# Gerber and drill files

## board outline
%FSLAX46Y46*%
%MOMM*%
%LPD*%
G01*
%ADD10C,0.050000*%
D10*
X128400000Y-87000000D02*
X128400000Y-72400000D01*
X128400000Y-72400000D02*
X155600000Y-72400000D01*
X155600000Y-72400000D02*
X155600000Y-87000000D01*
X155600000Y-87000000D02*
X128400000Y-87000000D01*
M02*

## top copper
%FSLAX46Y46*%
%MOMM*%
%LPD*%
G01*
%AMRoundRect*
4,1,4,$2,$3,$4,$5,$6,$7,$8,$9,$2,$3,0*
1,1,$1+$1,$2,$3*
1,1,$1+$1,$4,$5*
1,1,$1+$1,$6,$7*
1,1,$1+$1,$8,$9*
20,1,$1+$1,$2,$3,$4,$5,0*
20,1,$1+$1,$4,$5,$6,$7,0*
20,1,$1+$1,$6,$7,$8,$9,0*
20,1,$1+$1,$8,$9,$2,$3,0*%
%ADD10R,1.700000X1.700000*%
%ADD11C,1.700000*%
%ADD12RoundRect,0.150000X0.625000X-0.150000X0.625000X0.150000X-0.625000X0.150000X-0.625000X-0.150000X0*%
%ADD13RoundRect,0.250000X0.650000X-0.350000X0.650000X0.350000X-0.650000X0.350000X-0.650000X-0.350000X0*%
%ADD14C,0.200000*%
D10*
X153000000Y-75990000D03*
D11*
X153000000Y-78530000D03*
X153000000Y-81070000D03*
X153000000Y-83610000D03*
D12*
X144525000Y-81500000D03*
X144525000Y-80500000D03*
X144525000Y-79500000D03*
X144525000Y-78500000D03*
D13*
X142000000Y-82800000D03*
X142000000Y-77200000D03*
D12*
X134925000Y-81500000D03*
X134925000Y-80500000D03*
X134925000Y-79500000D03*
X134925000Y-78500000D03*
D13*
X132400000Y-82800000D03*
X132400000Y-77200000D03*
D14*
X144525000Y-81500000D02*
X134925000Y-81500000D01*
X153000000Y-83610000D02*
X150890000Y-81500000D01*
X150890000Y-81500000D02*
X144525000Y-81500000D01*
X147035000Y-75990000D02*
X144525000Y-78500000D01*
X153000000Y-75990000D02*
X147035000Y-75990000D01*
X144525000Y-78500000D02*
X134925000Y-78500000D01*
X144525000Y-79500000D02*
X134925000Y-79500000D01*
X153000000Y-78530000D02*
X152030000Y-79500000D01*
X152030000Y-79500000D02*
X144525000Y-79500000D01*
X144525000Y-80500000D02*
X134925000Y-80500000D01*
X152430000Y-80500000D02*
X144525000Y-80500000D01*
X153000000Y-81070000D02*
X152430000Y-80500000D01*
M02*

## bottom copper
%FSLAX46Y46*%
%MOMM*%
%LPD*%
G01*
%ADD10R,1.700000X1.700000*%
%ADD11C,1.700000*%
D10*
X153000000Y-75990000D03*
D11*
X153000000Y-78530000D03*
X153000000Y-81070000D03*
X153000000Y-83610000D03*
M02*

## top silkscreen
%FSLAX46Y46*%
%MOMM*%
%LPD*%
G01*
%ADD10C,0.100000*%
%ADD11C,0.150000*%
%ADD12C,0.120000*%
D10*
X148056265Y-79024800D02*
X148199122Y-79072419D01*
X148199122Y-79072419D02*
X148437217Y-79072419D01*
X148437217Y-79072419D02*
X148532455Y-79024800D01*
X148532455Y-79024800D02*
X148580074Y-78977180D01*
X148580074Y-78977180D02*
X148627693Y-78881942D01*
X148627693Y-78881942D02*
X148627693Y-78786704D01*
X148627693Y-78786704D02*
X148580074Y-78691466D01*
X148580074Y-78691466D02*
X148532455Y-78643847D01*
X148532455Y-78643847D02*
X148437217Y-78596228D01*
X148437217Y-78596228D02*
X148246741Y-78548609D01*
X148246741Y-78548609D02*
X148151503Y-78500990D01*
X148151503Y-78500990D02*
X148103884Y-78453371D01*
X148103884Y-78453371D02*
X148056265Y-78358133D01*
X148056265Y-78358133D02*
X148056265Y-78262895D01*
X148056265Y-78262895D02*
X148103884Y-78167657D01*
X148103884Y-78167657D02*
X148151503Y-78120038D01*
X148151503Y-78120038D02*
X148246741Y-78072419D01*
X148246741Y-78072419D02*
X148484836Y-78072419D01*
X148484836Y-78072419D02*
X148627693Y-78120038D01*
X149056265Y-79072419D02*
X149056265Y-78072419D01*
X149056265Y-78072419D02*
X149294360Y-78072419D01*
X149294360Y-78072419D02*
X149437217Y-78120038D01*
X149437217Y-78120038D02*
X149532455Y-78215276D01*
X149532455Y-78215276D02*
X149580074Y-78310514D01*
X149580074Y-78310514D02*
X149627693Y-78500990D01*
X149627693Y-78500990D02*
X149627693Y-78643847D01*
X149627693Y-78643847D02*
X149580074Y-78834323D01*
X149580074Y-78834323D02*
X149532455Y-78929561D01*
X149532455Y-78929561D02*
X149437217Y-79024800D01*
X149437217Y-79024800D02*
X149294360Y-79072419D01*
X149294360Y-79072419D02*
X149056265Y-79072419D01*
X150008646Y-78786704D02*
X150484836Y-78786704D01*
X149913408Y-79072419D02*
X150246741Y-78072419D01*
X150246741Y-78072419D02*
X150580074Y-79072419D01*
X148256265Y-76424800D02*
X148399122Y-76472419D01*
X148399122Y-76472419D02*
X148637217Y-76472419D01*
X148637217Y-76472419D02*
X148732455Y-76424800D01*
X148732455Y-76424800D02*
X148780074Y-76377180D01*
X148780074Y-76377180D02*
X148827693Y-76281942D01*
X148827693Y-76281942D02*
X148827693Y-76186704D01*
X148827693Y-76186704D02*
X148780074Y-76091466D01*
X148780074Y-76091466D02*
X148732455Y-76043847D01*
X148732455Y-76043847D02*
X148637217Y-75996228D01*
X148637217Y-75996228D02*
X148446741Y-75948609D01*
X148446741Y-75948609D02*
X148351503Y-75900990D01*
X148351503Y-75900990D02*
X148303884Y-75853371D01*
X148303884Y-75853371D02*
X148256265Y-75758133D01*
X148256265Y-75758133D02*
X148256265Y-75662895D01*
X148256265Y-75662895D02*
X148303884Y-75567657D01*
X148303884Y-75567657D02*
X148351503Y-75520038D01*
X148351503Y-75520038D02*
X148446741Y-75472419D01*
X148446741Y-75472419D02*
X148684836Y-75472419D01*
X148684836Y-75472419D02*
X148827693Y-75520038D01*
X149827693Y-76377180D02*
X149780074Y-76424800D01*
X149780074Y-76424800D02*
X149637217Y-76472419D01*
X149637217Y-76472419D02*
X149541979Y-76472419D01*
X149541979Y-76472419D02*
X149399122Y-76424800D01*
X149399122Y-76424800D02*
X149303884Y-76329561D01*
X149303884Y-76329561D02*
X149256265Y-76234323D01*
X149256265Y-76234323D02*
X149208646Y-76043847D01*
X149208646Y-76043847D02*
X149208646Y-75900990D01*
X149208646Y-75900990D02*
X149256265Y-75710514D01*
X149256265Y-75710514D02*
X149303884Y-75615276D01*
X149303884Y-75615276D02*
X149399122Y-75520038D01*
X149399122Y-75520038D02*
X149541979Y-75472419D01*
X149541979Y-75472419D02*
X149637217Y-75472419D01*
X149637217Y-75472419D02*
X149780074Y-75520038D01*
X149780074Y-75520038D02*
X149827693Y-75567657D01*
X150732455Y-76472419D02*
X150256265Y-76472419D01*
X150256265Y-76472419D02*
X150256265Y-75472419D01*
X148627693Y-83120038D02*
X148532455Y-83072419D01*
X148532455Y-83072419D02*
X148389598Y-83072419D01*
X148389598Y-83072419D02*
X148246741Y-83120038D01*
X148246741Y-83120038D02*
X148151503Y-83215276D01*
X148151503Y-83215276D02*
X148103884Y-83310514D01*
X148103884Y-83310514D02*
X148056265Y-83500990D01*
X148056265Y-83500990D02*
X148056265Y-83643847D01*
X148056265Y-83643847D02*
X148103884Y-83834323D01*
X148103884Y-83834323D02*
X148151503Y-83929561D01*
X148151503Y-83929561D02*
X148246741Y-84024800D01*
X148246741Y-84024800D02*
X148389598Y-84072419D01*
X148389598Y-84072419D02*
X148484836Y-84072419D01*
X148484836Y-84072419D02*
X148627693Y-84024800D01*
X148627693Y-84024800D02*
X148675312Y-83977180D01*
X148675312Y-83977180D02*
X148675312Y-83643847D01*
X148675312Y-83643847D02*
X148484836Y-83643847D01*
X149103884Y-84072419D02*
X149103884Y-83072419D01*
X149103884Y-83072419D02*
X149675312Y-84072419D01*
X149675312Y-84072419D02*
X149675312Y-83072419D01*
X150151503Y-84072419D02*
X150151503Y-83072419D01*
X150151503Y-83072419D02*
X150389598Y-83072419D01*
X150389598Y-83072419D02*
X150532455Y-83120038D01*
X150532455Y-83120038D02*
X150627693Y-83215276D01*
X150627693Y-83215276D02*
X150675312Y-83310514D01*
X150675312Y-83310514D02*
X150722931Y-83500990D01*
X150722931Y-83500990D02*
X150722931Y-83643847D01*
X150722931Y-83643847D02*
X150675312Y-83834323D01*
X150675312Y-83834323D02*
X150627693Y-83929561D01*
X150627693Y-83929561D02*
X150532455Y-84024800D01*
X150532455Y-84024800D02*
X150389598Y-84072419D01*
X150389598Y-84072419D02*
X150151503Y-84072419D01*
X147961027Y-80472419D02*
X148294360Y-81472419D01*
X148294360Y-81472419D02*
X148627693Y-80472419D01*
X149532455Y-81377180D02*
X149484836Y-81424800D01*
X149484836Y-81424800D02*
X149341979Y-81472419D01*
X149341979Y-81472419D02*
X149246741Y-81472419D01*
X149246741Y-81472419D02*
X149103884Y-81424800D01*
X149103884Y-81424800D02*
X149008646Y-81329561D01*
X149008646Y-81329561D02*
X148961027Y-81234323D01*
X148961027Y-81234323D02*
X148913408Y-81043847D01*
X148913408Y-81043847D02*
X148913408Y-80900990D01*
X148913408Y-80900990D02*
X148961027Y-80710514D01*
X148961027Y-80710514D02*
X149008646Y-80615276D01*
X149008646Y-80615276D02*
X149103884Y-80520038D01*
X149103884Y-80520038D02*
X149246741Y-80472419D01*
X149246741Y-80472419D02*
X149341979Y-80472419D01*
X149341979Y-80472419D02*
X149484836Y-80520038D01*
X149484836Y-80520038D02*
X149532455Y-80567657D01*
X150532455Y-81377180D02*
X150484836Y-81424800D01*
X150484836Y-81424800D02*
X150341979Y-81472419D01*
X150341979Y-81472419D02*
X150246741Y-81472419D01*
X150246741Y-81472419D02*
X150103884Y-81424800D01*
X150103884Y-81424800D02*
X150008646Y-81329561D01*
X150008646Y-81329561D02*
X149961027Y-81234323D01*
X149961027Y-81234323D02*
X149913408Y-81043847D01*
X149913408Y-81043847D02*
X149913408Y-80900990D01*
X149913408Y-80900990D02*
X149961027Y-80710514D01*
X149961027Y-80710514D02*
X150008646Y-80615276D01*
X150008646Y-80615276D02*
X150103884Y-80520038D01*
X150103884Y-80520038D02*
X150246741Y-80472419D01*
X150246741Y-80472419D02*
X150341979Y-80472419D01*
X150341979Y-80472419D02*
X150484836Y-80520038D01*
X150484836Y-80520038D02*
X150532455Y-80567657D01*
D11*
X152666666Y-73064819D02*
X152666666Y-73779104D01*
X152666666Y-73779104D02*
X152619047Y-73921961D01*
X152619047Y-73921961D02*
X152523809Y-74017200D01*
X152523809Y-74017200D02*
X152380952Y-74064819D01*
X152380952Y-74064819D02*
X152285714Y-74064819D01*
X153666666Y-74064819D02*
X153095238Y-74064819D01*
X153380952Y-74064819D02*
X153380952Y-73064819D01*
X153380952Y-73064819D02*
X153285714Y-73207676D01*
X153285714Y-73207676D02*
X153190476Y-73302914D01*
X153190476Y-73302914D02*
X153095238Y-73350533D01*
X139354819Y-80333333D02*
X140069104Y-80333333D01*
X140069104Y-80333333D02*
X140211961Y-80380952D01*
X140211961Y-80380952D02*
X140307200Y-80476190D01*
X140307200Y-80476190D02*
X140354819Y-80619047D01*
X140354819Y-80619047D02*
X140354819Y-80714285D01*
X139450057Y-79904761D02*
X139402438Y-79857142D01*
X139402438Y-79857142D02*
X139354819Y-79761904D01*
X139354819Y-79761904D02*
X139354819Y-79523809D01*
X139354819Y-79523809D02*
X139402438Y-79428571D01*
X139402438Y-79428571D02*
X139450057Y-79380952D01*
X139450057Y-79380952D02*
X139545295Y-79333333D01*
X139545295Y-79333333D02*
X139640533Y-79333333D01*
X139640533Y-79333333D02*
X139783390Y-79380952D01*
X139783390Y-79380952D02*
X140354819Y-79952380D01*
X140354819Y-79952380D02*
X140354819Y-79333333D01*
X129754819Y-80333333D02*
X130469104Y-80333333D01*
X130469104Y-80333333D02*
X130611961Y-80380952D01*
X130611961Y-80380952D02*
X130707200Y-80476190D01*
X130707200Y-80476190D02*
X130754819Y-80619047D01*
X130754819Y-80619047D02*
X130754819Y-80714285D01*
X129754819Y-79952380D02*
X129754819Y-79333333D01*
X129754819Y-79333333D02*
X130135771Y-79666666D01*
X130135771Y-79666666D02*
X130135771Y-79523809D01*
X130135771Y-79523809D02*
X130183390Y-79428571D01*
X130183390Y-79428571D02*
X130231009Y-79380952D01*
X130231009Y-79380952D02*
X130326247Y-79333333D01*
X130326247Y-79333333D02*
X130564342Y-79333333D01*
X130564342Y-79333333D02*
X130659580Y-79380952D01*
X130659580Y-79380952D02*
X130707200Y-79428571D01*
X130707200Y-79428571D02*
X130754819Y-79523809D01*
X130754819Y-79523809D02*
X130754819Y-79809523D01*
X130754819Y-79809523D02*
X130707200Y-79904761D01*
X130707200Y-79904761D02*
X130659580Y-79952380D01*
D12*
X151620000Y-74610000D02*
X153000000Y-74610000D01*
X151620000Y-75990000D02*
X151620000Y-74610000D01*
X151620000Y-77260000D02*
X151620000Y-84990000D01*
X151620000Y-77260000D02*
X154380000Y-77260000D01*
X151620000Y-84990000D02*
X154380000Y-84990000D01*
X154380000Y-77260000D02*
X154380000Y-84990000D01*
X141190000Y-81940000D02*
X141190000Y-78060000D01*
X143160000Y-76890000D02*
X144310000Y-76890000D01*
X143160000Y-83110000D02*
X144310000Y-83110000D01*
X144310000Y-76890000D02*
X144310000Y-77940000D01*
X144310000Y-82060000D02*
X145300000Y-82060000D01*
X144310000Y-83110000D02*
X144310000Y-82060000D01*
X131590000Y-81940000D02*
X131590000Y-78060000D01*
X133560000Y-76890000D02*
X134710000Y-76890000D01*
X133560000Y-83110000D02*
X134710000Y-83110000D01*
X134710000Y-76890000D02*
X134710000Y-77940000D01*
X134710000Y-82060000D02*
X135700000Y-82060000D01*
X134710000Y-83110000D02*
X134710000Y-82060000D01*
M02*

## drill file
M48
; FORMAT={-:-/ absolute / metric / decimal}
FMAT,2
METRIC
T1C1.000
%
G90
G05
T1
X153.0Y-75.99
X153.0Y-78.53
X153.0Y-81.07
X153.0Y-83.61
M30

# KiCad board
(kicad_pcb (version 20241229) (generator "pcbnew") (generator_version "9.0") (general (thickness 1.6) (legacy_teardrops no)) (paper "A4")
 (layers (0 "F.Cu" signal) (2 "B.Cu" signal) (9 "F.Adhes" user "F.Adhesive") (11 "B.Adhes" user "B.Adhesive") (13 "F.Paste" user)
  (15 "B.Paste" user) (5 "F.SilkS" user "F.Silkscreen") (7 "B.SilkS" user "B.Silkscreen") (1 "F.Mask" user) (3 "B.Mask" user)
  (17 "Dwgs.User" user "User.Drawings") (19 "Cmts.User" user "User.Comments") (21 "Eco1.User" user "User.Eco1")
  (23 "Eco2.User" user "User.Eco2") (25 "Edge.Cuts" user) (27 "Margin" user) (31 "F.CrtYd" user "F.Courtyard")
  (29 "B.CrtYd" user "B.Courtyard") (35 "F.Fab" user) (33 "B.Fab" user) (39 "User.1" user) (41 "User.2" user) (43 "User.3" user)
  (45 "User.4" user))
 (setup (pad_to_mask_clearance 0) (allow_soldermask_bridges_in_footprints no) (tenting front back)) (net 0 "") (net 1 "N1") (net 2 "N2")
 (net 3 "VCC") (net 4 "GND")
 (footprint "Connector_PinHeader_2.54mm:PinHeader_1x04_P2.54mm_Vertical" (layer "F.Cu") (at 153 75.99)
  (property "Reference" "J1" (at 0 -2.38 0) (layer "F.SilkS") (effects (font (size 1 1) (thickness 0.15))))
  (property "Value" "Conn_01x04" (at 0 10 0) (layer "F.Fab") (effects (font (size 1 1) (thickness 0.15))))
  (fp_line (start -1.38 -1.38) (end 0 -1.38) (stroke (width 0.12) (type solid)) (layer "F.SilkS"))
  (fp_line (start -1.38 0) (end -1.38 -1.38) (stroke (width 0.12) (type solid)) (layer "F.SilkS"))
  (fp_line (start -1.38 1.27) (end -1.38 9) (stroke (width 0.12) (type solid)) (layer "F.SilkS"))
  (fp_line (start -1.38 1.27) (end 1.38 1.27) (stroke (width 0.12) (type solid)) (layer "F.SilkS"))
  (fp_line (start -1.38 9) (end 1.38 9) (stroke (width 0.12) (type solid)) (layer "F.SilkS"))
  (fp_line (start 1.38 1.27) (end 1.38 9) (stroke (width 0.12) (type solid)) (layer "F.SilkS"))
  (pad "1" thru_hole rect (at 0 0) (size 1.7 1.7) (drill 1) (layers "*.Cu" "*.Mask") (remove_unused_layers no) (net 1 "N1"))
  (pad "2" thru_hole circle (at 0 2.54) (size 1.7 1.7) (drill 1) (layers "*.Cu" "*.Mask") (remove_unused_layers no) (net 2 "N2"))
  (pad "3" thru_hole circle (at 0 5.08) (size 1.7 1.7) (drill 1) (layers "*.Cu" "*.Mask") (remove_unused_layers no) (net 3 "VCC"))
  (pad "4" thru_hole circle (at 0 7.62) (size 1.7 1.7) (drill 1) (layers "*.Cu" "*.Mask") (remove_unused_layers no) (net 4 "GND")))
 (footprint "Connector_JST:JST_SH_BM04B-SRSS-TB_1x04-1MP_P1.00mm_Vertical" (layer "F.Cu") (at 143.2 80 90)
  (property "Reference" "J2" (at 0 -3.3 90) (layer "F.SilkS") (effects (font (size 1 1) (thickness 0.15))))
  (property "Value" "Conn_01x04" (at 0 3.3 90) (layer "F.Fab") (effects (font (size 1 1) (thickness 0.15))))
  (fp_line (start -1.94 -2.01) (end 1.94 -2.01) (stroke (width 0.12) (type solid)) (layer "F.SilkS"))
  (fp_line (start 3.11 -0.04) (end 3.11 1.11) (stroke (width 0.12) (type solid)) (layer "F.SilkS"))
  (fp_line (start -3.11 -0.04) (end -3.11 1.11) (stroke (width 0.12) (type solid)) (layer "F.SilkS"))
  (fp_line (start 3.11 1.11) (end 2.06 1.11) (stroke (width 0.12) (type solid)) (layer "F.SilkS"))
  (fp_line (start -2.06 1.11) (end -2.06 2.1) (stroke (width 0.12) (type solid)) (layer "F.SilkS"))
  (fp_line (start -3.11 1.11) (end -2.06 1.11) (stroke (width 0.12) (type solid)) (layer "F.SilkS"))
  (pad "1" smd roundrect (at -1.5 1.325 90) (size 0.6 1.55) (layers "F.Cu" "F.Mask" "F.Paste") (roundrect_rratio 0.25) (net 4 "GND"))
  (pad "2" smd roundrect (at -0.5 1.325 90) (size 0.6 1.55) (layers "F.Cu" "F.Mask" "F.Paste") (roundrect_rratio 0.25) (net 3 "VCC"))
  (pad "3" smd roundrect (at 0.5 1.325 90) (size 0.6 1.55) (layers "F.Cu" "F.Mask" "F.Paste") (roundrect_rratio 0.25) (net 2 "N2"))
  (pad "4" smd roundrect (at 1.5 1.325 90) (size 0.6 1.55) (layers "F.Cu" "F.Mask" "F.Paste") (roundrect_rratio 0.25) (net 1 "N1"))
  (pad "MP" smd roundrect (at -2.8 -1.2 90) (size 1.2 1.8) (layers "F.Cu" "F.Mask" "F.Paste") (roundrect_rratio 0.208333))
  (pad "MP" smd roundrect (at 2.8 -1.2 90) (size 1.2 1.8) (layers "F.Cu" "F.Mask" "F.Paste") (roundrect_rratio 0.208333)))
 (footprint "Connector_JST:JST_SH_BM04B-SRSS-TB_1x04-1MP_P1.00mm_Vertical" (layer "F.Cu") (at 133.6 80 90)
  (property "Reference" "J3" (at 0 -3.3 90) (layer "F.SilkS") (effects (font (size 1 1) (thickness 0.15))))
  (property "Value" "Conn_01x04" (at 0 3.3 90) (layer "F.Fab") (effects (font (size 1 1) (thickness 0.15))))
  (fp_line (start -1.94 -2.01) (end 1.94 -2.01) (stroke (width 0.12) (type solid)) (layer "F.SilkS"))
  (fp_line (start 3.11 -0.04) (end 3.11 1.11) (stroke (width 0.12) (type solid)) (layer "F.SilkS"))
  (fp_line (start -3.11 -0.04) (end -3.11 1.11) (stroke (width 0.12) (type solid)) (layer "F.SilkS"))
  (fp_line (start 3.11 1.11) (end 2.06 1.11) (stroke (width 0.12) (type solid)) (layer "F.SilkS"))
  (fp_line (start -2.06 1.11) (end -2.06 2.1) (stroke (width 0.12) (type solid)) (layer "F.SilkS"))
  (fp_line (start -3.11 1.11) (end -2.06 1.11) (stroke (width 0.12) (type solid)) (layer "F.SilkS"))
  (pad "1" smd roundrect (at -1.5 1.325 90) (size 0.6 1.55) (layers "F.Cu" "F.Mask" "F.Paste") (roundrect_rratio 0.25) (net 4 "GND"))
  (pad "2" smd roundrect (at -0.5 1.325 90) (size 0.6 1.55) (layers "F.Cu" "F.Mask" "F.Paste") (roundrect_rratio 0.25) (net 3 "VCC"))
  (pad "3" smd roundrect (at 0.5 1.325 90) (size 0.6 1.55) (layers "F.Cu" "F.Mask" "F.Paste") (roundrect_rratio 0.25) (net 2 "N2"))
  (pad "4" smd roundrect (at 1.5 1.325 90) (size 0.6 1.55) (layers "F.Cu" "F.Mask" "F.Paste") (roundrect_rratio 0.25) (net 1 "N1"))
  (pad "MP" smd roundrect (at -2.8 -1.2 90) (size 1.2 1.8) (layers "F.Cu" "F.Mask" "F.Paste") (roundrect_rratio 0.208333))
  (pad "MP" smd roundrect (at 2.8 -1.2 90) (size 1.2 1.8) (layers "F.Cu" "F.Mask" "F.Paste") (roundrect_rratio 0.208333)))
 (gr_line (start 128.4 87) (end 128.4 72.4) (stroke (width 0.05) (type default)) (layer "Edge.Cuts"))
 (gr_line (start 128.4 72.4) (end 155.6 72.4) (stroke (width 0.05) (type default)) (layer "Edge.Cuts"))
 (gr_line (start 155.6 72.4) (end 155.6 87) (stroke (width 0.05) (type default)) (layer "Edge.Cuts"))
 (gr_line (start 155.6 87) (end 128.4 87) (stroke (width 0.05) (type default)) (layer "Edge.Cuts"))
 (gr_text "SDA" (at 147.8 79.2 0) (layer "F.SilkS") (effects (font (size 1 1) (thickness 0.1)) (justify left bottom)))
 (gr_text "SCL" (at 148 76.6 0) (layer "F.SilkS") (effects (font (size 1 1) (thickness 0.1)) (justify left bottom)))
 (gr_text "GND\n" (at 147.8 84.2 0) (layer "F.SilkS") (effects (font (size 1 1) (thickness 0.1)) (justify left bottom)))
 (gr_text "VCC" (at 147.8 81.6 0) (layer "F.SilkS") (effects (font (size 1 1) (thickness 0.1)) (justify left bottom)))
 (segment (start 144.525 81.5) (end 134.925 81.5) (width 0.2) (layer "F.Cu") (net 4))
 (segment (start 153 83.61) (end 150.89 81.5) (width 0.2) (layer "F.Cu") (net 4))
 (segment (start 150.89 81.5) (end 144.525 81.5) (width 0.2) (layer "F.Cu") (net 4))
 (segment (start 147.035 75.99) (end 144.525 78.5) (width 0.2) (layer "F.Cu") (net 1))
 (segment (start 153 75.99) (end 147.035 75.99) (width 0.2) (layer "F.Cu") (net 1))
 (segment (start 144.525 78.5) (end 134.925 78.5) (width 0.2) (layer "F.Cu") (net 1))
 (segment (start 144.525 79.5) (end 134.925 79.5) (width 0.2) (layer "F.Cu") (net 2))
 (segment (start 153 78.53) (end 152.03 79.5) (width 0.2) (layer "F.Cu") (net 2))
 (segment (start 152.03 79.5) (end 144.525 79.5) (width 0.2) (layer "F.Cu") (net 2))
 (segment (start 144.525 80.5) (end 134.925 80.5) (width 0.2) (layer "F.Cu") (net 3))
 (segment (start 152.43 80.5) (end 144.525 80.5) (width 0.2) (layer "F.Cu") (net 3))
 (segment (start 153 81.07) (end 152.43 80.5) (width 0.2) (layer "F.Cu") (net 3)))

